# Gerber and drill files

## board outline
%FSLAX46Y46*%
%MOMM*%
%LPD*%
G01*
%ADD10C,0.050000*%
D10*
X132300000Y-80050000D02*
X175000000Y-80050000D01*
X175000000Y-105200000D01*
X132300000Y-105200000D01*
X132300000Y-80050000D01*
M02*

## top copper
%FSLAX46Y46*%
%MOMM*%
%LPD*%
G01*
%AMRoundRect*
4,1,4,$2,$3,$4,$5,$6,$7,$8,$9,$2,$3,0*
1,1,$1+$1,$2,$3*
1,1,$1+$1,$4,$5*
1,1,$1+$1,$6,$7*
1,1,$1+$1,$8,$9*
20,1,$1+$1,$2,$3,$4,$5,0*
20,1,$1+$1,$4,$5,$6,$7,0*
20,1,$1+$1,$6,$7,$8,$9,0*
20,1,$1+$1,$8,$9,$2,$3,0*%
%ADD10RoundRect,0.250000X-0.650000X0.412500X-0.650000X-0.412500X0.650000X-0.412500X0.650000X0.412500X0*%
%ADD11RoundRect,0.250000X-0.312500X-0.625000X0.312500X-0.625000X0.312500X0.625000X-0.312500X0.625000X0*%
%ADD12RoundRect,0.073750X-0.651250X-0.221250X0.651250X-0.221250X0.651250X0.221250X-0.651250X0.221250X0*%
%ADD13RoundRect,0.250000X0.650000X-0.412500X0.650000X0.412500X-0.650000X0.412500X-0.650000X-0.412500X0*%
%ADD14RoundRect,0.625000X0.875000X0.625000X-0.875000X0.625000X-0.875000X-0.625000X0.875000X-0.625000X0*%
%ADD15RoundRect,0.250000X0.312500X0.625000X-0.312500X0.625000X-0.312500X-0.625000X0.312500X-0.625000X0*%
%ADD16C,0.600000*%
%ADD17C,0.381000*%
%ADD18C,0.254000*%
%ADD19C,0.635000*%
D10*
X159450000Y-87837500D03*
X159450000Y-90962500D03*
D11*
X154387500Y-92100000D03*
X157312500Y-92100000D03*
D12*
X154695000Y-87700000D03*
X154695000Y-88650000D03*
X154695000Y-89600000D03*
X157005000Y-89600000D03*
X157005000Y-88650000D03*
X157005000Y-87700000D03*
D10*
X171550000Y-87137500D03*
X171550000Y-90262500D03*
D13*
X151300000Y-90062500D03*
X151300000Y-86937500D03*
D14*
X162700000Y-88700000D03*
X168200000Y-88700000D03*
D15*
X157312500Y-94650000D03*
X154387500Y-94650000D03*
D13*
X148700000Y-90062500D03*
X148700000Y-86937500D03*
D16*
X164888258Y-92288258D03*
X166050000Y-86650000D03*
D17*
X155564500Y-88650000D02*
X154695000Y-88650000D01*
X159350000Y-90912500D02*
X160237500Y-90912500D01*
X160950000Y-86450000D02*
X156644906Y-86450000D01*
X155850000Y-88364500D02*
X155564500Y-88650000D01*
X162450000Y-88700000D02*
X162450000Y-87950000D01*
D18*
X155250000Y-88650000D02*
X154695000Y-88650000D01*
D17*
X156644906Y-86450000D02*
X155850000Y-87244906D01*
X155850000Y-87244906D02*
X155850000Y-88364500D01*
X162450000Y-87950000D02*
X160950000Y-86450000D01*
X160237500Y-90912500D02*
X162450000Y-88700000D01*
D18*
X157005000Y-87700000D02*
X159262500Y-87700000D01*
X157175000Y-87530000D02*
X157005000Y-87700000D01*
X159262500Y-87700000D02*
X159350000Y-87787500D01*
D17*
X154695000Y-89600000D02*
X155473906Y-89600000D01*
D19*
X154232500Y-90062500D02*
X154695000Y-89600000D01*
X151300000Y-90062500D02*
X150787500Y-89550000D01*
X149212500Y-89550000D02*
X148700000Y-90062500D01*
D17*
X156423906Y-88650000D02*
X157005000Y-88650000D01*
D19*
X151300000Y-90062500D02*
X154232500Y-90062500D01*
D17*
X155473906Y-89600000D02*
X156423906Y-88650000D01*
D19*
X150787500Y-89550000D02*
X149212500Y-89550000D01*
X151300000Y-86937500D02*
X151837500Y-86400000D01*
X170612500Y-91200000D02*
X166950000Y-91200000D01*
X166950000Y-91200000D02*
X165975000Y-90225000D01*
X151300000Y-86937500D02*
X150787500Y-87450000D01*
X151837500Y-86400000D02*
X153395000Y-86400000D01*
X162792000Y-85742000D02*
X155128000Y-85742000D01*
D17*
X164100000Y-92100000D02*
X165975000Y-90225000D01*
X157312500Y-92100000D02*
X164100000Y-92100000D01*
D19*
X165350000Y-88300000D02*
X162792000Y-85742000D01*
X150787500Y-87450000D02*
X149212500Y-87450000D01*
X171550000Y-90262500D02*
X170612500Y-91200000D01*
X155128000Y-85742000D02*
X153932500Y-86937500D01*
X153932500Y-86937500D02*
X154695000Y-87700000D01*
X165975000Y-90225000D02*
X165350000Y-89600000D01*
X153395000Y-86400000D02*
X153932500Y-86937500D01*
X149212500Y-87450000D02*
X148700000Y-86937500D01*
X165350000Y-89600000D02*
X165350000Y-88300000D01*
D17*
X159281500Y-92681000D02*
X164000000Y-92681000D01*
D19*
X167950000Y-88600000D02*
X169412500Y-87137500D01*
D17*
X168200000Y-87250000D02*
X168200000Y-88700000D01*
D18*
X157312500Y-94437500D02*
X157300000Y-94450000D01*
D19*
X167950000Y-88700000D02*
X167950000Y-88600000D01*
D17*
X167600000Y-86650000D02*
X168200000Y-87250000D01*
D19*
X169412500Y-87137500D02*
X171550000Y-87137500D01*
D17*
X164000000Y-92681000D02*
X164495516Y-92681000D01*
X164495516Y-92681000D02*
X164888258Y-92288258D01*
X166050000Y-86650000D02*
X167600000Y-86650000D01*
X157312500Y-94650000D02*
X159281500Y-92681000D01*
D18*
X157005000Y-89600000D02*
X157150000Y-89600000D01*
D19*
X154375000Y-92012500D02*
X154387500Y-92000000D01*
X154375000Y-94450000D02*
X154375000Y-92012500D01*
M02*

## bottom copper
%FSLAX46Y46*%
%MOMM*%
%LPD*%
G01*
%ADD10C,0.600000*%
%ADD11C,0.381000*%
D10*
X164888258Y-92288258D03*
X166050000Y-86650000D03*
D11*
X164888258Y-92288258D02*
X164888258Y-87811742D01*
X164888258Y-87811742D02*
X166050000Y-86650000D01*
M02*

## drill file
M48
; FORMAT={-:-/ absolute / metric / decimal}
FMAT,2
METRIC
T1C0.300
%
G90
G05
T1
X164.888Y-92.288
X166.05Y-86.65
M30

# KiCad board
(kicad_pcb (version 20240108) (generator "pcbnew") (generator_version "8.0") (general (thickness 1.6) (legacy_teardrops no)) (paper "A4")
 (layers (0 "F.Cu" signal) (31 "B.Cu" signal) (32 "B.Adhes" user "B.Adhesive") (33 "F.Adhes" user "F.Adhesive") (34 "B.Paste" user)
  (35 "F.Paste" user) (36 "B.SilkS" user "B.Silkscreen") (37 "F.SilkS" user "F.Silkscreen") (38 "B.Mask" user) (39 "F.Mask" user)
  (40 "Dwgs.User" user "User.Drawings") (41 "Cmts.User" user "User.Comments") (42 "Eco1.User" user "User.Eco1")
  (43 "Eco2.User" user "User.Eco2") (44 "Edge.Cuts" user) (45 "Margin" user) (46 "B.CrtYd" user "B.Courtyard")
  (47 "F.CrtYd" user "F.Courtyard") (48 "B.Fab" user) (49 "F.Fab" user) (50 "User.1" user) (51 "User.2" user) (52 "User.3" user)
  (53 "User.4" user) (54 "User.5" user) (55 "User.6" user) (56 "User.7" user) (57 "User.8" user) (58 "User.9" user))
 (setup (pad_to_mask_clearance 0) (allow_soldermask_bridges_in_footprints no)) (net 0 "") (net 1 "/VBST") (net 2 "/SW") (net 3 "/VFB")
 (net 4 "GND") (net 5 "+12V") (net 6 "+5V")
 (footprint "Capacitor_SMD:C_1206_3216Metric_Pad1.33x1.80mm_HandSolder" (layer "F.Cu") (at 159.45 89.4 -90)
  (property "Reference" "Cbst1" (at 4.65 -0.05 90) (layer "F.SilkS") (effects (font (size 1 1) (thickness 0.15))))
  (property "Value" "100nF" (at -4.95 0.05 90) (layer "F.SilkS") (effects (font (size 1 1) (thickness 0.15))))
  (pad "1" smd roundrect (at -1.5625 0 270) (size 1.325 1.8) (layers "F.Cu" "F.Paste" "F.Mask") (roundrect_rratio 0.188679) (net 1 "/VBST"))
  (pad "2" smd roundrect (at 1.5625 0 270) (size 1.325 1.8) (layers "F.Cu" "F.Paste" "F.Mask") (roundrect_rratio 0.188679) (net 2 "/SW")))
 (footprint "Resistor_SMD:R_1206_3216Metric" (layer "F.Cu") (at 155.85 92.1)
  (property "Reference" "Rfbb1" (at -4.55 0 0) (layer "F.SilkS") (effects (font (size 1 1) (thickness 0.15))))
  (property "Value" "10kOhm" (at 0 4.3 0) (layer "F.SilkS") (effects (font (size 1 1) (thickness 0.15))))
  (pad "1" smd roundrect (at -1.4625 0) (size 1.125 1.75) (layers "F.Cu" "F.Paste" "F.Mask") (roundrect_rratio 0.222222) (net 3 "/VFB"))
  (pad "2" smd roundrect (at 1.4625 0) (size 1.125 1.75) (layers "F.Cu" "F.Paste" "F.Mask") (roundrect_rratio 0.222222) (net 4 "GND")))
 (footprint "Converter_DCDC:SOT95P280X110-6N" (layer "F.Cu") (at 155.85 88.65)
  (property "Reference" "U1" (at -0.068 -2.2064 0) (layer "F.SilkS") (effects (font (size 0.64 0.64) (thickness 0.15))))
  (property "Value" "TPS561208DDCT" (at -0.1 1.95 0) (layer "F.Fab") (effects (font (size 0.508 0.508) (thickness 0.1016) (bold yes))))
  (pad "1" smd roundrect (at -1.155 -0.95) (size 1.45 0.59) (layers "F.Cu" "F.Paste" "F.Mask") (roundrect_rratio 0.125) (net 4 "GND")
   (solder_mask_margin 0.102))
  (pad "2" smd roundrect (at -1.155 0) (size 1.45 0.59) (layers "F.Cu" "F.Paste" "F.Mask") (roundrect_rratio 0.125) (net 2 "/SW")
   (solder_mask_margin 0.102))
  (pad "3" smd roundrect (at -1.155 0.95) (size 1.45 0.59) (layers "F.Cu" "F.Paste" "F.Mask") (roundrect_rratio 0.125) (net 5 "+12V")
   (solder_mask_margin 0.102))
  (pad "4" smd roundrect (at 1.155 0.95) (size 1.45 0.59) (layers "F.Cu" "F.Paste" "F.Mask") (roundrect_rratio 0.125) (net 3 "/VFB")
   (solder_mask_margin 0.102))
  (pad "5" smd roundrect (at 1.155 0) (size 1.45 0.59) (layers "F.Cu" "F.Paste" "F.Mask") (roundrect_rratio 0.125) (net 5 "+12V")
   (solder_mask_margin 0.102))
  (pad "6" smd roundrect (at 1.155 -0.95) (size 1.45 0.59) (layers "F.Cu" "F.Paste" "F.Mask") (roundrect_rratio 0.125) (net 1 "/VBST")
   (solder_mask_margin 0.102)))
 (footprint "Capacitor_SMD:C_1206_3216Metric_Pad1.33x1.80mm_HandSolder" (layer "F.Cu") (at 171.55 88.7 -90)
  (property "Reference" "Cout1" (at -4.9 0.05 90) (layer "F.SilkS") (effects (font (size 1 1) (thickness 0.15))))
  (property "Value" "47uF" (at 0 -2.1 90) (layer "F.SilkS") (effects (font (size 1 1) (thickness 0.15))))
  (pad "1" smd roundrect (at -1.5625 0 270) (size 1.325 1.8) (layers "F.Cu" "F.Paste" "F.Mask") (roundrect_rratio 0.188679) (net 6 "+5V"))
  (pad "2" smd roundrect (at 1.5625 0 270) (size 1.325 1.8) (layers "F.Cu" "F.Paste" "F.Mask") (roundrect_rratio 0.188679) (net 4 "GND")))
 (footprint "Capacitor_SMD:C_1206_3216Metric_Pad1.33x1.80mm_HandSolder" (layer "F.Cu") (at 151.3 88.5 90)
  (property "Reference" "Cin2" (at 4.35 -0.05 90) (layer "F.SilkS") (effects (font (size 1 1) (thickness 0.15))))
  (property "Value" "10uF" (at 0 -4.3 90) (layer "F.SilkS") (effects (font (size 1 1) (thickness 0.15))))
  (pad "1" smd roundrect (at -1.5625 0 90) (size 1.325 1.8) (layers "F.Cu" "F.Paste" "F.Mask") (roundrect_rratio 0.188679) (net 5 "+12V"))
  (pad "2" smd roundrect (at 1.5625 0 90) (size 1.325 1.8) (layers "F.Cu" "F.Paste" "F.Mask") (roundrect_rratio 0.188679) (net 4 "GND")))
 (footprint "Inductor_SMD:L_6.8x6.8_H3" (layer "F.Cu") (at 165.45 88.7 180)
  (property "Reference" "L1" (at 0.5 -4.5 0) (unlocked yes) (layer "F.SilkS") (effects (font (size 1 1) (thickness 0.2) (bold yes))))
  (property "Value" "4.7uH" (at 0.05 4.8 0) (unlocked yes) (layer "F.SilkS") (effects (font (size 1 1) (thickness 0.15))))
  (pad "1" smd roundrect (at 2.75 0 180) (size 3 2.5) (layers "F.Cu" "F.Paste" "F.Mask") (roundrect_rratio 0.25) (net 2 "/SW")
   (thermal_bridge_angle 45))
  (pad "2" smd roundrect (at -2.75 0 180) (size 3 2.5) (layers "F.Cu" "F.Paste" "F.Mask") (roundrect_rratio 0.25) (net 6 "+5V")
   (thermal_bridge_angle 45)))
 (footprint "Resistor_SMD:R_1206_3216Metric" (layer "F.Cu") (at 155.85 94.65 180)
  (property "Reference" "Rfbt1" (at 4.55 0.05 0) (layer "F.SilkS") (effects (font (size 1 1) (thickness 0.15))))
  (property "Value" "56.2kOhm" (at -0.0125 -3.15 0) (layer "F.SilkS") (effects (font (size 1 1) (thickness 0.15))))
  (pad "1" smd roundrect (at -1.4625 0 180) (size 1.125 1.75) (layers "F.Cu" "F.Paste" "F.Mask") (roundrect_rratio 0.222222) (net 6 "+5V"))
  (pad "2" smd roundrect (at 1.4625 0 180) (size 1.125 1.75) (layers "F.Cu" "F.Paste" "F.Mask") (roundrect_rratio 0.222222) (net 3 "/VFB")))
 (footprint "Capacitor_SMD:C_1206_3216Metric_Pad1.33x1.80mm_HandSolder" (layer "F.Cu") (at 148.7 88.5 90)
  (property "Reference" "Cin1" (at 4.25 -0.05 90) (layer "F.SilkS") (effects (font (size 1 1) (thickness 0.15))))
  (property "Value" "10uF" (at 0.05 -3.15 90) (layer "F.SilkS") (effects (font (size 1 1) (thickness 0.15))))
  (pad "1" smd roundrect (at -1.5625 0 90) (size 1.325 1.8) (layers "F.Cu" "F.Paste" "F.Mask") (roundrect_rratio 0.188679) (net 5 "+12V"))
  (pad "2" smd roundrect (at 1.5625 0 90) (size 1.325 1.8) (layers "F.Cu" "F.Paste" "F.Mask") (roundrect_rratio 0.188679) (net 4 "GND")))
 (gr_rect (start 132.3 80.05) (end 175 105.2) (stroke (width 0.05) (type default)) (fill none) (layer "Edge.Cuts"))
 (segment (start 155.5645 88.65) (end 154.695 88.65) (width 0.381) (layer "F.Cu") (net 2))
 (segment (start 159.35 90.9125) (end 160.2375 90.9125) (width 0.381) (layer "F.Cu") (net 2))
 (segment (start 160.95 86.45) (end 156.644906 86.45) (width 0.381) (layer "F.Cu") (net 2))
 (segment (start 155.85 88.3645) (end 155.5645 88.65) (width 0.381) (layer "F.Cu") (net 2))
 (segment (start 162.45 88.7) (end 162.45 87.95) (width 0.381) (layer "F.Cu") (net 2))
 (segment (start 155.25 88.65) (end 154.695 88.65) (width 0.254) (layer "F.Cu") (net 2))
 (segment (start 156.644906 86.45) (end 155.85 87.244906) (width 0.381) (layer "F.Cu") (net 2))
 (segment (start 155.85 87.244906) (end 155.85 88.3645) (width 0.381) (layer "F.Cu") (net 2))
 (segment (start 162.45 87.95) (end 160.95 86.45) (width 0.381) (layer "F.Cu") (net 2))
 (segment (start 160.2375 90.9125) (end 162.45 88.7) (width 0.381) (layer "F.Cu") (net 2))
 (segment (start 157.005 87.7) (end 159.2625 87.7) (width 0.254) (layer "F.Cu") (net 1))
 (segment (start 157.175 87.53) (end 157.005 87.7) (width 0.254) (layer "F.Cu") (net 1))
 (segment (start 159.2625 87.7) (end 159.35 87.7875) (width 0.254) (layer "F.Cu") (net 1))
 (segment (start 154.695 89.6) (end 155.473906 89.6) (width 0.381) (layer "F.Cu") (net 5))
 (segment (start 154.2325 90.0625) (end 154.695 89.6) (width 0.635) (layer "F.Cu") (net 5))
 (segment (start 151.3 90.0625) (end 150.7875 89.55) (width 0.635) (layer "F.Cu") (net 5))
 (segment (start 149.2125 89.55) (end 148.7 90.0625) (width 0.635) (layer "F.Cu") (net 5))
 (segment (start 156.423906 88.65) (end 157.005 88.65) (width 0.381) (layer "F.Cu") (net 5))
 (segment (start 151.3 90.0625) (end 154.2325 90.0625) (width 0.635) (layer "F.Cu") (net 5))
 (segment (start 155.473906 89.6) (end 156.423906 88.65) (width 0.381) (layer "F.Cu") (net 5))
 (segment (start 150.7875 89.55) (end 149.2125 89.55) (width 0.635) (layer "F.Cu") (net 5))
 (segment (start 151.3 86.9375) (end 151.8375 86.4) (width 0.635) (layer "F.Cu") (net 4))
 (segment (start 170.6125 91.2) (end 166.95 91.2) (width 0.635) (layer "F.Cu") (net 4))
 (segment (start 166.95 91.2) (end 165.975 90.225) (width 0.635) (layer "F.Cu") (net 4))
 (segment (start 151.3 86.9375) (end 150.7875 87.45) (width 0.635) (layer "F.Cu") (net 4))
 (segment (start 151.8375 86.4) (end 153.395 86.4) (width 0.635) (layer "F.Cu") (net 4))
 (segment (start 162.792 85.742) (end 155.128 85.742) (width 0.635) (layer "F.Cu") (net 4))
 (segment (start 164.1 92.1) (end 165.975 90.225) (width 0.381) (layer "F.Cu") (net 4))
 (segment (start 157.3125 92.1) (end 164.1 92.1) (width 0.381) (layer "F.Cu") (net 4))
 (segment (start 165.35 88.3) (end 162.792 85.742) (width 0.635) (layer "F.Cu") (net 4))
 (segment (start 150.7875 87.45) (end 149.2125 87.45) (width 0.635) (layer "F.Cu") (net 4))
 (segment (start 171.55 90.2625) (end 170.6125 91.2) (width 0.635) (layer "F.Cu") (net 4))
 (segment (start 155.128 85.742) (end 153.9325 86.9375) (width 0.635) (layer "F.Cu") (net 4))
 (segment (start 153.9325 86.9375) (end 154.695 87.7) (width 0.635) (layer "F.Cu") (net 4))
 (segment (start 165.975 90.225) (end 165.35 89.6) (width 0.635) (layer "F.Cu") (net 4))
 (segment (start 153.395 86.4) (end 153.9325 86.9375) (width 0.635) (layer "F.Cu") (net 4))
 (segment (start 149.2125 87.45) (end 148.7 86.9375) (width 0.635) (layer "F.Cu") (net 4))
 (segment (start 165.35 89.6) (end 165.35 88.3) (width 0.635) (layer "F.Cu") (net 4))
 (segment (start 159.2815 92.681) (end 164 92.681) (width 0.381) (layer "F.Cu") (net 6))
 (segment (start 167.95 88.6) (end 169.4125 87.1375) (width 0.635) (layer "F.Cu") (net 6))
 (segment (start 168.2 87.25) (end 168.2 88.7) (width 0.381) (layer "F.Cu") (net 6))
 (segment (start 157.3125 94.4375) (end 157.3 94.45) (width 0.254) (layer "F.Cu") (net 6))
 (segment (start 167.95 88.7) (end 167.95 88.6) (width 0.635) (layer "F.Cu") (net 6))
 (segment (start 167.6 86.65) (end 168.2 87.25) (width 0.381) (layer "F.Cu") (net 6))
 (segment (start 169.4125 87.1375) (end 171.55 87.1375) (width 0.635) (layer "F.Cu") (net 6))
 (segment (start 164 92.681) (end 164.495516 92.681) (width 0.381) (layer "F.Cu") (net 6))
 (segment (start 164.495516 92.681) (end 164.888258 92.288258) (width 0.381) (layer "F.Cu") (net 6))
 (segment (start 166.05 86.65) (end 167.6 86.65) (width 0.381) (layer "F.Cu") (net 6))
 (segment (start 157.3125 94.65) (end 159.2815 92.681) (width 0.381) (layer "F.Cu") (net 6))
 (via (at 164.888258 92.288258) (size 0.6) (drill 0.3) (layers "F.Cu" "B.Cu") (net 6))
 (via (at 166.05 86.65) (size 0.6) (drill 0.3) (layers "F.Cu" "B.Cu") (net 6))
 (segment (start 164.888258 92.288258) (end 164.888258 87.811742) (width 0.381) (layer "B.Cu") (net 6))
 (segment (start 164.888258 87.811742) (end 166.05 86.65) (width 0.381) (layer "B.Cu") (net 6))
 (segment (start 157.005 89.6) (end 157.15 89.6) (width 0.254) (layer "F.Cu") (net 3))
 (segment (start 154.375 92.0125) (end 154.3875 92) (width 0.635) (layer "F.Cu") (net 3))
 (segment (start 154.375 94.45) (end 154.375 92.0125) (width 0.635) (layer "F.Cu") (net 3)))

